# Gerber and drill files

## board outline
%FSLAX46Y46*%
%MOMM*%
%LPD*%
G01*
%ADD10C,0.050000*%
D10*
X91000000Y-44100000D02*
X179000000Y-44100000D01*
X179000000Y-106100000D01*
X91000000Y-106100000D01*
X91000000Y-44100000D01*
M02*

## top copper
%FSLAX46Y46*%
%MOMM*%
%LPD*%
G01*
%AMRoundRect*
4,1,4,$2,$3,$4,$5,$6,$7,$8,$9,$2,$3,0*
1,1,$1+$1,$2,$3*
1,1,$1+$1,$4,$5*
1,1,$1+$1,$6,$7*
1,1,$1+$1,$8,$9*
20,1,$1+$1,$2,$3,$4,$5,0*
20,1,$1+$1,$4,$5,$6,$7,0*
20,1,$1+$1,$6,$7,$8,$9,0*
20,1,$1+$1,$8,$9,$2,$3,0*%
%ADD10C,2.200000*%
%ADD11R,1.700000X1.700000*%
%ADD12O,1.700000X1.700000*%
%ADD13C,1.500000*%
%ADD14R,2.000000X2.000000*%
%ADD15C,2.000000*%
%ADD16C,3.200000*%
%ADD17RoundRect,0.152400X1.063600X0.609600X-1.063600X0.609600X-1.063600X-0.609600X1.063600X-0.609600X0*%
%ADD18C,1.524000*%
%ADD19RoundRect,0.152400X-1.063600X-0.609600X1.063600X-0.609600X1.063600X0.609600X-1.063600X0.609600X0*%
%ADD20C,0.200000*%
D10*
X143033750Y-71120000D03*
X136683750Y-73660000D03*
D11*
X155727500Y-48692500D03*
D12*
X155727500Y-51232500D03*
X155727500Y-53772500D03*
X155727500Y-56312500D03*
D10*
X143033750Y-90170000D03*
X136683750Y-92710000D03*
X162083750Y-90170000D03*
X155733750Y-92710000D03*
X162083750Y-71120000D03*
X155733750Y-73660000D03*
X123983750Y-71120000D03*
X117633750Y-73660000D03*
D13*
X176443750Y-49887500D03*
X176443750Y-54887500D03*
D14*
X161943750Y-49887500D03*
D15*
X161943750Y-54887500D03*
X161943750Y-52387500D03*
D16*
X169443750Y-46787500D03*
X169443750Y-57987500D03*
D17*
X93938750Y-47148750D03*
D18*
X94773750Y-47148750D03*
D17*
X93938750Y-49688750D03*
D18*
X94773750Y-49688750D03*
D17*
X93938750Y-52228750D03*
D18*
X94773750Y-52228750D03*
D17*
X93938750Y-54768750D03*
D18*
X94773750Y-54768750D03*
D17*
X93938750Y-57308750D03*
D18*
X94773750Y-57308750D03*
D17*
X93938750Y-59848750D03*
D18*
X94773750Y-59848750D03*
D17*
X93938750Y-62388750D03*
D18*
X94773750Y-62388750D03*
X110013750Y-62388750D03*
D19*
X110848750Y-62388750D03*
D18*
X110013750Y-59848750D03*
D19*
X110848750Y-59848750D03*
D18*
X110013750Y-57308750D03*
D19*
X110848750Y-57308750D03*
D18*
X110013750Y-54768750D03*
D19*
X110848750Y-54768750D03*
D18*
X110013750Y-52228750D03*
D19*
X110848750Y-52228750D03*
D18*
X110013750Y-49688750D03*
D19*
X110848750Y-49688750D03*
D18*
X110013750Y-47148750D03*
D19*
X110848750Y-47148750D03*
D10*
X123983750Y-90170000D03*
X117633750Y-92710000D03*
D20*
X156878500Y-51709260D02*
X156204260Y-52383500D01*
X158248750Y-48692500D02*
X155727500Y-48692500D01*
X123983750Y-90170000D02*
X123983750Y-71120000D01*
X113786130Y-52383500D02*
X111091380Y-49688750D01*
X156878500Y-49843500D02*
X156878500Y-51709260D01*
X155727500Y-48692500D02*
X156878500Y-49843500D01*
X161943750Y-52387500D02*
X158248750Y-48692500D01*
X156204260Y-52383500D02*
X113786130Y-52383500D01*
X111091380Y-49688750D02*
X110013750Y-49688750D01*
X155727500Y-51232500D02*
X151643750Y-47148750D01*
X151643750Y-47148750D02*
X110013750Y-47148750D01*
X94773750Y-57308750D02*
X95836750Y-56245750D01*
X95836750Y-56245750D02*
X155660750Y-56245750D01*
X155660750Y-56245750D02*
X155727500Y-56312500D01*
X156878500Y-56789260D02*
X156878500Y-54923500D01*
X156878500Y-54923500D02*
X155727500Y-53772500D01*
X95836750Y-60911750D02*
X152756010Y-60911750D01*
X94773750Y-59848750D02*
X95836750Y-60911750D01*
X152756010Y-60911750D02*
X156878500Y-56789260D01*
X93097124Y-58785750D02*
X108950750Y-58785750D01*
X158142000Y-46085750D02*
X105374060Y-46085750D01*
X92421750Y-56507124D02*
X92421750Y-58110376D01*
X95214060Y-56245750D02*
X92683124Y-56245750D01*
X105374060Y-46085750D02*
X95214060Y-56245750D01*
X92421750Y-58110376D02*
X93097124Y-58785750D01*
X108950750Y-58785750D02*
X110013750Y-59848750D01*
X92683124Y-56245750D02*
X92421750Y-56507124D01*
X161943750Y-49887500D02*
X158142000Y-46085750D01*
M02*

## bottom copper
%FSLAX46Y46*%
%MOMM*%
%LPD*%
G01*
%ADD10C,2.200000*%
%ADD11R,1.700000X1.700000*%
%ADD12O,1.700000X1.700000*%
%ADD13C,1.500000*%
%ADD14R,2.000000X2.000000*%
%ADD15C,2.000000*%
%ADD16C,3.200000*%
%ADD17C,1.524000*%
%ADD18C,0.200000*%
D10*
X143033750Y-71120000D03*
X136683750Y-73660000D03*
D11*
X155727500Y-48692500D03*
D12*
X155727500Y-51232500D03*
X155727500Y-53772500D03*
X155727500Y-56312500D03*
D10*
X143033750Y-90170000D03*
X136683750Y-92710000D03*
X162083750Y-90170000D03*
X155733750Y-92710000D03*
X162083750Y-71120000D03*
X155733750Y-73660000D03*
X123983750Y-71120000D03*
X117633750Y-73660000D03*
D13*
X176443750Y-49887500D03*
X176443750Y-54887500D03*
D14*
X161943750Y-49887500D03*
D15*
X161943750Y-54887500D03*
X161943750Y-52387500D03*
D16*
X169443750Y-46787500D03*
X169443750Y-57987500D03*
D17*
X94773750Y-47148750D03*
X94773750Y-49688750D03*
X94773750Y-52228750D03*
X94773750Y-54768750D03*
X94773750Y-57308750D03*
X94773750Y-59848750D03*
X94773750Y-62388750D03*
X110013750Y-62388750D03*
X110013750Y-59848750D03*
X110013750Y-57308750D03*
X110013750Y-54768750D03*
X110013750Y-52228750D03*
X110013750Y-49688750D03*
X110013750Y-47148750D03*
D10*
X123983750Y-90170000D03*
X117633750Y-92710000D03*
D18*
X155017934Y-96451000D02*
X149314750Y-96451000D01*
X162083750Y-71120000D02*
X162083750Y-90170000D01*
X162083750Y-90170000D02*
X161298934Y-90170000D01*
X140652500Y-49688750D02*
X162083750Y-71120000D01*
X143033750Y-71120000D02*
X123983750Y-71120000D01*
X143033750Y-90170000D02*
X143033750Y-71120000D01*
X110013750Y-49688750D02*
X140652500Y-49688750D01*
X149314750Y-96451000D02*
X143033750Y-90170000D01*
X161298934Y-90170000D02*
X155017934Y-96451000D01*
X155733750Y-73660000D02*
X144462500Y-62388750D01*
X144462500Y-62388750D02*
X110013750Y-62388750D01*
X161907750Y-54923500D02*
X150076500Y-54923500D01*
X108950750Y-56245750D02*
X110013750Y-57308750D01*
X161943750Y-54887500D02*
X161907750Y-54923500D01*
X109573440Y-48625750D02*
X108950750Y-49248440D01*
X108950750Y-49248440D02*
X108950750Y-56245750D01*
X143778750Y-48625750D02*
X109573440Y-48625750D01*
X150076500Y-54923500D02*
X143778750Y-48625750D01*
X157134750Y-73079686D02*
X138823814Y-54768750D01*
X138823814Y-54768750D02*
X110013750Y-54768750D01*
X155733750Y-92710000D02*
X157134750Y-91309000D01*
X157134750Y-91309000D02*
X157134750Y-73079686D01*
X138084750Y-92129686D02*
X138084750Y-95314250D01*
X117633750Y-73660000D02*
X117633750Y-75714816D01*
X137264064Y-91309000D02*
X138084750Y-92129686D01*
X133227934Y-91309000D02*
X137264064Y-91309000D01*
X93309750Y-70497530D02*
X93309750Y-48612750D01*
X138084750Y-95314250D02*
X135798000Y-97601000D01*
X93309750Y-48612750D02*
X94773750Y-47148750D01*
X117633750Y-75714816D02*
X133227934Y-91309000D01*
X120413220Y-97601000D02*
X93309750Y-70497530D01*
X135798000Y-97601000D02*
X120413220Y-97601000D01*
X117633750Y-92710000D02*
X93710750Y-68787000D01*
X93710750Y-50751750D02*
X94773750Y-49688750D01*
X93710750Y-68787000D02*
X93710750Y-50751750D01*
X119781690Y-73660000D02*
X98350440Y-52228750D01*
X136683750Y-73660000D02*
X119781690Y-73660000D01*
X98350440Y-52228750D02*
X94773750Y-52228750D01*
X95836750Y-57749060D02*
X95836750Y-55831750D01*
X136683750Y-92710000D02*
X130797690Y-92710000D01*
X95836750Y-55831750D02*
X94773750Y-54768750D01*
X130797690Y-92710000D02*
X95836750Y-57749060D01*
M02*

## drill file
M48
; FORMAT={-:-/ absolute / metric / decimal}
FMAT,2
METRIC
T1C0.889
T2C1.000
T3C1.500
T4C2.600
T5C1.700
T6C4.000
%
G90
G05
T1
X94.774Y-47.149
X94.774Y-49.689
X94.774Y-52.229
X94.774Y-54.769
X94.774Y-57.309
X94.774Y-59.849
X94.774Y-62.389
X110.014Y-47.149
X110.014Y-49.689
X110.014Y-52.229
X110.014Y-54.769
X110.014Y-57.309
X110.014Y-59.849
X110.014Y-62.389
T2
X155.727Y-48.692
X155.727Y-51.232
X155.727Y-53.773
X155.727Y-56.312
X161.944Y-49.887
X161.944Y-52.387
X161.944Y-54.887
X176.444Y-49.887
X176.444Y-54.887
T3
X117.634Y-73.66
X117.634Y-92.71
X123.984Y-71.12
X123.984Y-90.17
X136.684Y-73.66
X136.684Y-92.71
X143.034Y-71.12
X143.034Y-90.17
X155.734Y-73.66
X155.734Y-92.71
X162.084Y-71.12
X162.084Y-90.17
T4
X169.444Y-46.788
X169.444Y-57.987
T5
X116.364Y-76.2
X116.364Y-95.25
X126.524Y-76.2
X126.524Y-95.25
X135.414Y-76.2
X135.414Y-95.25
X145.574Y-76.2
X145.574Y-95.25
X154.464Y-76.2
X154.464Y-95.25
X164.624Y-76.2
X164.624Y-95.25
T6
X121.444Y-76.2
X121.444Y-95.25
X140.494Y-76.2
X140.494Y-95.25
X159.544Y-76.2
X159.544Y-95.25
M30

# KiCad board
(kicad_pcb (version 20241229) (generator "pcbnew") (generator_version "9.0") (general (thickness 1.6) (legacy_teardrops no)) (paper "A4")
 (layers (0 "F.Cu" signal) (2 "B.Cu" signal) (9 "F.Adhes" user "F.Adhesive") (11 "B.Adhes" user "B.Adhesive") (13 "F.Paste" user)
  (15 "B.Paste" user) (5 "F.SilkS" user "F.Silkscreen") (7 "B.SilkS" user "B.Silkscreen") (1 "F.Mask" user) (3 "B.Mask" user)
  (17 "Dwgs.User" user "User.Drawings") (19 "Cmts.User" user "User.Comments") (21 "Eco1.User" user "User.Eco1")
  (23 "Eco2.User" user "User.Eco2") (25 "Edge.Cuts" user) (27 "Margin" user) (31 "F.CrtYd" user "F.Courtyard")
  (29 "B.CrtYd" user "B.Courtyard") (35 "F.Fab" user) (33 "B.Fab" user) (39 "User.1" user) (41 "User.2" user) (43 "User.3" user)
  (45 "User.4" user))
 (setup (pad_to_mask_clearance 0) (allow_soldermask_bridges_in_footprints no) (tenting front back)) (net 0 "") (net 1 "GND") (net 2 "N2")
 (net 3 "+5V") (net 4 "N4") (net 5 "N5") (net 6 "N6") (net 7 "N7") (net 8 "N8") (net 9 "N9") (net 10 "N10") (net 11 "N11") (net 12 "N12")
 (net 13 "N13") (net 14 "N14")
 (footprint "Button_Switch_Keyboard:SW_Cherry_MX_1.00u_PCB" (layer "F.Cu") (at 143.03375 71.12)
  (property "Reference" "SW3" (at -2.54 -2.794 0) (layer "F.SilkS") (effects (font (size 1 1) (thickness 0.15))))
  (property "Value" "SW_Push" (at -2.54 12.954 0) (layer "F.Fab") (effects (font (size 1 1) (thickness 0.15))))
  (pad "" np_thru_hole circle (at -7.62 5.08) (size 1.7 1.7) (drill 1.7) (layers "*.Cu" "*.Mask"))
  (pad "" np_thru_hole circle (at -2.54 5.08) (size 4 4) (drill 4) (layers "*.Cu" "*.Mask"))
  (pad "" np_thru_hole circle (at 2.54 5.08) (size 1.7 1.7) (drill 1.7) (layers "*.Cu" "*.Mask"))
  (pad "1" thru_hole circle (at 0 0) (size 2.2 2.2) (drill 1.5) (layers "*.Cu" "*.Mask") (remove_unused_layers no) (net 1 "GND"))
  (pad "2" thru_hole circle (at -6.35 2.54) (size 2.2 2.2) (drill 1.5) (layers "*.Cu" "*.Mask") (remove_unused_layers no) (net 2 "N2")))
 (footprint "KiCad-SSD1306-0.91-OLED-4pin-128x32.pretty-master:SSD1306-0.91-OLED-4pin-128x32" (layer "F.Cu") (at 119.2275 46.5025)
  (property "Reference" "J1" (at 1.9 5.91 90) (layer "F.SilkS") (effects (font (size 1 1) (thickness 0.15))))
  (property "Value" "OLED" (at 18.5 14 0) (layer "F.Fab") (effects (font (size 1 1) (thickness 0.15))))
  (pad "1" thru_hole rect (at 36.5 2.19) (size 1.7 1.7) (drill 1) (layers "*.Cu" "*.Mask") (remove_unused_layers no) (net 1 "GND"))
  (pad "2" thru_hole oval (at 36.5 4.73) (size 1.7 1.7) (drill 1) (layers "*.Cu" "*.Mask") (remove_unused_layers no) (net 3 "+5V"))
  (pad "3" thru_hole oval (at 36.5 7.27) (size 1.7 1.7) (drill 1) (layers "*.Cu" "*.Mask") (remove_unused_layers no) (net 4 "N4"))
  (pad "4" thru_hole oval (at 36.5 9.81) (size 1.7 1.7) (drill 1) (layers "*.Cu" "*.Mask") (remove_unused_layers no) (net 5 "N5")))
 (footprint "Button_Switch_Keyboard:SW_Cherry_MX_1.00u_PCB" (layer "F.Cu") (at 143.03375 90.17)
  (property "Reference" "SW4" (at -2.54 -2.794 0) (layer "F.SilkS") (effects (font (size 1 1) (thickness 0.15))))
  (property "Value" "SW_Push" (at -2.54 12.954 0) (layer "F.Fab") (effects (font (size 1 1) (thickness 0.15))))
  (pad "" np_thru_hole circle (at -7.62 5.08) (size 1.7 1.7) (drill 1.7) (layers "*.Cu" "*.Mask"))
  (pad "" np_thru_hole circle (at -2.54 5.08) (size 4 4) (drill 4) (layers "*.Cu" "*.Mask"))
  (pad "" np_thru_hole circle (at 2.54 5.08) (size 1.7 1.7) (drill 1.7) (layers "*.Cu" "*.Mask"))
  (pad "1" thru_hole circle (at 0 0) (size 2.2 2.2) (drill 1.5) (layers "*.Cu" "*.Mask") (remove_unused_layers no) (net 1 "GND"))
  (pad "2" thru_hole circle (at -6.35 2.54) (size 2.2 2.2) (drill 1.5) (layers "*.Cu" "*.Mask") (remove_unused_layers no) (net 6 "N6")))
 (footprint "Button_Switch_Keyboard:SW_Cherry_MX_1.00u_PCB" (layer "F.Cu") (at 162.08375 90.17)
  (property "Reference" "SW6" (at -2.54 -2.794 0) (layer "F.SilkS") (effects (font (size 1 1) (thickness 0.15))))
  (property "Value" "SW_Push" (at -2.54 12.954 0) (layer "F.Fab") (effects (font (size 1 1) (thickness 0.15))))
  (pad "" np_thru_hole circle (at -7.62 5.08) (size 1.7 1.7) (drill 1.7) (layers "*.Cu" "*.Mask"))
  (pad "" np_thru_hole circle (at -2.54 5.08) (size 4 4) (drill 4) (layers "*.Cu" "*.Mask"))
  (pad "" np_thru_hole circle (at 2.54 5.08) (size 1.7 1.7) (drill 1.7) (layers "*.Cu" "*.Mask"))
  (pad "1" thru_hole circle (at 0 0) (size 2.2 2.2) (drill 1.5) (layers "*.Cu" "*.Mask") (remove_unused_layers no) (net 1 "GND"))
  (pad "2" thru_hole circle (at -6.35 2.54) (size 2.2 2.2) (drill 1.5) (layers "*.Cu" "*.Mask") (remove_unused_layers no) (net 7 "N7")))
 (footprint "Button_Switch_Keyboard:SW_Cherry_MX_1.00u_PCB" (layer "F.Cu") (at 162.08375 71.12)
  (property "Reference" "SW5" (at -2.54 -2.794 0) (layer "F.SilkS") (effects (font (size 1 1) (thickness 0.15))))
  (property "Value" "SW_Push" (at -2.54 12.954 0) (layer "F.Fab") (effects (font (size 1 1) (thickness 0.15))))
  (pad "" np_thru_hole circle (at -7.62 5.08) (size 1.7 1.7) (drill 1.7) (layers "*.Cu" "*.Mask"))
  (pad "" np_thru_hole circle (at -2.54 5.08) (size 4 4) (drill 4) (layers "*.Cu" "*.Mask"))
  (pad "" np_thru_hole circle (at 2.54 5.08) (size 1.7 1.7) (drill 1.7) (layers "*.Cu" "*.Mask"))
  (pad "1" thru_hole circle (at 0 0) (size 2.2 2.2) (drill 1.5) (layers "*.Cu" "*.Mask") (remove_unused_layers no) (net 1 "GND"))
  (pad "2" thru_hole circle (at -6.35 2.54) (size 2.2 2.2) (drill 1.5) (layers "*.Cu" "*.Mask") (remove_unused_layers no) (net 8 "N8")))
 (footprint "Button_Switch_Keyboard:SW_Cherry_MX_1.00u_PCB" (layer "F.Cu") (at 123.98375 71.12)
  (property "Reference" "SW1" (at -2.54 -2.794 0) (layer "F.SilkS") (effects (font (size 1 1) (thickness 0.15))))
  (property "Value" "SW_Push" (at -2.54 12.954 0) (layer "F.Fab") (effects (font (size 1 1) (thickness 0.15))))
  (pad "" np_thru_hole circle (at -7.62 5.08) (size 1.7 1.7) (drill 1.7) (layers "*.Cu" "*.Mask"))
  (pad "" np_thru_hole circle (at -2.54 5.08) (size 4 4) (drill 4) (layers "*.Cu" "*.Mask"))
  (pad "" np_thru_hole circle (at 2.54 5.08) (size 1.7 1.7) (drill 1.7) (layers "*.Cu" "*.Mask"))
  (pad "1" thru_hole circle (at 0 0) (size 2.2 2.2) (drill 1.5) (layers "*.Cu" "*.Mask") (remove_unused_layers no) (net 1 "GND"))
  (pad "2" thru_hole circle (at -6.35 2.54) (size 2.2 2.2) (drill 1.5) (layers "*.Cu" "*.Mask") (remove_unused_layers no) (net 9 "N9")))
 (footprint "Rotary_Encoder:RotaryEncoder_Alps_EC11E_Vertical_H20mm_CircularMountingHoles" (layer "F.Cu") (at 161.94375 49.8875)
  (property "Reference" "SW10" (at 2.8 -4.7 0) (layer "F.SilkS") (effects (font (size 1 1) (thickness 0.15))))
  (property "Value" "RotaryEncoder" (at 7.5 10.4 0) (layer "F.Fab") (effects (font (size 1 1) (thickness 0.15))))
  (pad "" thru_hole circle (at 14.5 0) (size 1.5 1.5) (drill 1) (layers "*.Cu" "*.Mask") (remove_unused_layers no))
  (pad "" thru_hole circle (at 14.5 5) (size 1.5 1.5) (drill 1) (layers "*.Cu" "*.Mask") (remove_unused_layers no))
  (pad "A" thru_hole rect (at 0 0) (size 2 2) (drill 1) (layers "*.Cu" "*.Mask") (remove_unused_layers no) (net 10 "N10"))
  (pad "B" thru_hole circle (at 0 5) (size 2 2) (drill 1) (layers "*.Cu" "*.Mask") (remove_unused_layers no) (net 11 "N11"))
  (pad "C" thru_hole circle (at 0 2.5) (size 2 2) (drill 1) (layers "*.Cu" "*.Mask") (remove_unused_layers no) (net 1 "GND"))
  (pad "MP" thru_hole circle (at 7.5 -3.1) (size 3.2 3.2) (drill 2.6) (layers "*.Cu" "*.Mask") (remove_unused_layers no))
  (pad "MP" thru_hole circle (at 7.5 8.1) (size 3.2 3.2) (drill 2.6) (layers "*.Cu" "*.Mask") (remove_unused_layers no)))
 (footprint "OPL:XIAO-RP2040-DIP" (layer "F.Cu") (at 102.39375 54.76875)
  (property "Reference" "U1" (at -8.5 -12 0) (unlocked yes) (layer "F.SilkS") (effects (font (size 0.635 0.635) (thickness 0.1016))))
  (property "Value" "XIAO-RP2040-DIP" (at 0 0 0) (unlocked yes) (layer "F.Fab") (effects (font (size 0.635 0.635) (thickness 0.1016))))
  (pad "1" smd roundrect (at -8.455 -7.62 180) (size 2.432 1.524) (layers "F.Cu" "F.Mask") (roundrect_rratio 0.1) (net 9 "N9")
   (thermal_bridge_angle 45))
  (pad "1" thru_hole circle (at -7.62 -7.62 180) (size 1.524 1.524) (drill 0.889) (layers "*.Cu" "*.Mask") (remove_unused_layers no)
   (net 9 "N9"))
  (pad "2" smd roundrect (at -8.455 -5.08 180) (size 2.432 1.524) (layers "F.Cu" "F.Mask") (roundrect_rratio 0.1) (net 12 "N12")
   (thermal_bridge_angle 45))
  (pad "2" thru_hole circle (at -7.62 -5.08 180) (size 1.524 1.524) (drill 0.889) (layers "*.Cu" "*.Mask") (remove_unused_layers no)
   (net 12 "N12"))
  (pad "3" smd roundrect (at -8.455 -2.54 180) (size 2.432 1.524) (layers "F.Cu" "F.Mask") (roundrect_rratio 0.1) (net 2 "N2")
   (thermal_bridge_angle 45))
  (pad "3" thru_hole circle (at -7.62 -2.54 180) (size 1.524 1.524) (drill 0.889) (layers "*.Cu" "*.Mask") (remove_unused_layers no)
   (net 2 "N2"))
  (pad "4" smd roundrect (at -8.455 0 180) (size 2.432 1.524) (layers "F.Cu" "F.Mask") (roundrect_rratio 0.1) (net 6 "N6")
   (thermal_bridge_angle 45))
  (pad "4" thru_hole circle (at -7.62 0 180) (size 1.524 1.524) (drill 0.889) (layers "*.Cu" "*.Mask") (remove_unused_layers no)
   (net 6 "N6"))
  (pad "5" smd roundrect (at -8.455 2.54 180) (size 2.432 1.524) (layers "F.Cu" "F.Mask") (roundrect_rratio 0.1) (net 5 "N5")
   (thermal_bridge_angle 45))
  (pad "5" thru_hole circle (at -7.62 2.54 180) (size 1.524 1.524) (drill 0.889) (layers "*.Cu" "*.Mask") (remove_unused_layers no)
   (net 5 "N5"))
  (pad "6" smd roundrect (at -8.455 5.08 180) (size 2.432 1.524) (layers "F.Cu" "F.Mask") (roundrect_rratio 0.1) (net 4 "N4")
   (thermal_bridge_angle 45))
  (pad "6" thru_hole circle (at -7.62 5.08 180) (size 1.524 1.524) (drill 0.889) (layers "*.Cu" "*.Mask") (remove_unused_layers no)
   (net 4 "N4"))
  (pad "7" smd roundrect (at -8.455 7.62 180) (size 2.432 1.524) (layers "F.Cu" "F.Mask") (roundrect_rratio 0.1) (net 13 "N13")
   (thermal_bridge_angle 45))
  (pad "7" thru_hole circle (at -7.62 7.62 180) (size 1.524 1.524) (drill 0.889) (layers "*.Cu" "*.Mask") (remove_unused_layers no)
   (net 13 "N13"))
  (pad "8" thru_hole circle (at 7.62 7.62) (size 1.524 1.524) (drill 0.889) (layers "*.Cu" "*.Mask") (remove_unused_layers no) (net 8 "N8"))
  (pad "8" smd roundrect (at 8.455 7.62) (size 2.432 1.524) (layers "F.Cu" "F.Mask") (roundrect_rratio 0.1) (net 8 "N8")
   (thermal_bridge_angle 45))
  (pad "9" thru_hole circle (at 7.62 5.08) (size 1.524 1.524) (drill 0.889) (layers "*.Cu" "*.Mask") (remove_unused_layers no)
   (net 10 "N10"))
  (pad "9" smd roundrect (at 8.455 5.08) (size 2.432 1.524) (layers "F.Cu" "F.Mask") (roundrect_rratio 0.1) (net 10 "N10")
   (thermal_bridge_angle 45))
  (pad "10" thru_hole circle (at 7.62 2.54) (size 1.524 1.524) (drill 0.889) (layers "*.Cu" "*.Mask") (remove_unused_layers no)
   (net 11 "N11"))
  (pad "10" smd roundrect (at 8.455 2.54) (size 2.432 1.524) (layers "F.Cu" "F.Mask") (roundrect_rratio 0.1) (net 11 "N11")
   (thermal_bridge_angle 45))
  (pad "11" thru_hole circle (at 7.62 0) (size 1.524 1.524) (drill 0.889) (layers "*.Cu" "*.Mask") (remove_unused_layers no) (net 7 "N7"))
  (pad "11" smd roundrect (at 8.455 0) (size 2.432 1.524) (layers "F.Cu" "F.Mask") (roundrect_rratio 0.1) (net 7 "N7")
   (thermal_bridge_angle 45))
  (pad "12" thru_hole circle (at 7.62 -2.54) (size 1.524 1.524) (drill 0.889) (layers "*.Cu" "*.Mask") (remove_unused_layers no)
   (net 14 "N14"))
  (pad "12" smd roundrect (at 8.455 -2.54) (size 2.432 1.524) (layers "F.Cu" "F.Mask") (roundrect_rratio 0.1) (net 14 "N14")
   (thermal_bridge_angle 45))
  (pad "13" thru_hole circle (at 7.62 -5.08) (size 1.524 1.524) (drill 0.889) (layers "*.Cu" "*.Mask") (remove_unused_layers no)
   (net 1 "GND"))
  (pad "13" smd roundrect (at 8.455 -5.08) (size 2.432 1.524) (layers "F.Cu" "F.Mask") (roundrect_rratio 0.1) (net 1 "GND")
   (thermal_bridge_angle 45))
  (pad "14" thru_hole circle (at 7.62 -7.62) (size 1.524 1.524) (drill 0.889) (layers "*.Cu" "*.Mask") (remove_unused_layers no)
   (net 3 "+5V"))
  (pad "14" smd roundrect (at 8.455 -7.62) (size 2.432 1.524) (layers "F.Cu" "F.Mask") (roundrect_rratio 0.1) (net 3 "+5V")
   (thermal_bridge_angle 45)))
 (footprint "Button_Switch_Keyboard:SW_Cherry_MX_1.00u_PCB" (layer "F.Cu") (at 123.98375 90.17)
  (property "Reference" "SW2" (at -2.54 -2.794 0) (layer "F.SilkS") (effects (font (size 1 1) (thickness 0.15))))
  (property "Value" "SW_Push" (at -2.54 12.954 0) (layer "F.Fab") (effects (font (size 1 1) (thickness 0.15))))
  (pad "" np_thru_hole circle (at -7.62 5.08) (size 1.7 1.7) (drill 1.7) (layers "*.Cu" "*.Mask"))
  (pad "" np_thru_hole circle (at -2.54 5.08) (size 4 4) (drill 4) (layers "*.Cu" "*.Mask"))
  (pad "" np_thru_hole circle (at 2.54 5.08) (size 1.7 1.7) (drill 1.7) (layers "*.Cu" "*.Mask"))
  (pad "1" thru_hole circle (at 0 0) (size 2.2 2.2) (drill 1.5) (layers "*.Cu" "*.Mask") (remove_unused_layers no) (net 1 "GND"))
  (pad "2" thru_hole circle (at -6.35 2.54) (size 2.2 2.2) (drill 1.5) (layers "*.Cu" "*.Mask") (remove_unused_layers no) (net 12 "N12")))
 (gr_rect (start 91 44.1) (end 179 106.1) (stroke (width 0.05) (type default)) (fill no) (layer "Edge.Cuts"))
 (segment (start 156.8785 51.70926) (end 156.20426 52.3835) (width 0.2) (layer "F.Cu") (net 1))
 (segment (start 158.24875 48.6925) (end 155.7275 48.6925) (width 0.2) (layer "F.Cu") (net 1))
 (segment (start 123.98375 90.17) (end 123.98375 71.12) (width 0.2) (layer "F.Cu") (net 1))
 (segment (start 113.78613 52.3835) (end 111.09138 49.68875) (width 0.2) (layer "F.Cu") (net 1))
 (segment (start 156.8785 49.8435) (end 156.8785 51.70926) (width 0.2) (layer "F.Cu") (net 1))
 (segment (start 155.7275 48.6925) (end 156.8785 49.8435) (width 0.2) (layer "F.Cu") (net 1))
 (segment (start 161.94375 52.3875) (end 158.24875 48.6925) (width 0.2) (layer "F.Cu") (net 1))
 (segment (start 156.20426 52.3835) (end 113.78613 52.3835) (width 0.2) (layer "F.Cu") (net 1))
 (segment (start 111.09138 49.68875) (end 110.01375 49.68875) (width 0.2) (layer "F.Cu") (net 1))
 (segment (start 155.017934 96.451) (end 149.31475 96.451) (width 0.2) (layer "B.Cu") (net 1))
 (segment (start 162.08375 71.12) (end 162.08375 90.17) (width 0.2) (layer "B.Cu") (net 1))
 (segment (start 162.08375 90.17) (end 161.298934 90.17) (width 0.2) (layer "B.Cu") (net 1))
 (segment (start 140.6525 49.68875) (end 162.08375 71.12) (width 0.2) (layer "B.Cu") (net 1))
 (segment (start 143.03375 71.12) (end 123.98375 71.12) (width 0.2) (layer "B.Cu") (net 1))
 (segment (start 143.03375 90.17) (end 143.03375 71.12) (width 0.2) (layer "B.Cu") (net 1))
 (segment (start 110.01375 49.68875) (end 140.6525 49.68875) (width 0.2) (layer "B.Cu") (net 1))
 (segment (start 149.31475 96.451) (end 143.03375 90.17) (width 0.2) (layer "B.Cu") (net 1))
 (segment (start 161.298934 90.17) (end 155.017934 96.451) (width 0.2) (layer "B.Cu") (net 1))
 (segment (start 155.7275 51.2325) (end 151.64375 47.14875) (width 0.2) (layer "F.Cu") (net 3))
 (segment (start 151.64375 47.14875) (end 110.01375 47.14875) (width 0.2) (layer "F.Cu") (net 3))
 (segment (start 155.73375 73.66) (end 144.4625 62.38875) (width 0.2) (layer "B.Cu") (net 8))
 (segment (start 144.4625 62.38875) (end 110.01375 62.38875) (width 0.2) (layer "B.Cu") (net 8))
 (segment (start 94.77375 57.30875) (end 95.83675 56.24575) (width 0.2) (layer "F.Cu") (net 5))
 (segment (start 95.83675 56.24575) (end 155.66075 56.24575) (width 0.2) (layer "F.Cu") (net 5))
 (segment (start 155.66075 56.24575) (end 155.7275 56.3125) (width 0.2) (layer "F.Cu") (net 5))
 (segment (start 161.90775 54.9235) (end 150.0765 54.9235) (width 0.2) (layer "B.Cu") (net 11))
 (segment (start 108.95075 56.24575) (end 110.01375 57.30875) (width 0.2) (layer "B.Cu") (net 11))
 (segment (start 161.94375 54.8875) (end 161.90775 54.9235) (width 0.2) (layer "B.Cu") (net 11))
 (segment (start 109.57344 48.62575) (end 108.95075 49.24844) (width 0.2) (layer "B.Cu") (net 11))
 (segment (start 108.95075 49.24844) (end 108.95075 56.24575) (width 0.2) (layer "B.Cu") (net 11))
 (segment (start 143.77875 48.62575) (end 109.57344 48.62575) (width 0.2) (layer "B.Cu") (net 11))
 (segment (start 150.0765 54.9235) (end 143.77875 48.62575) (width 0.2) (layer "B.Cu") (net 11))
 (segment (start 157.13475 73.079686) (end 138.823814 54.76875) (width 0.2) (layer "B.Cu") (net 7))
 (segment (start 138.823814 54.76875) (end 110.01375 54.76875) (width 0.2) (layer "B.Cu") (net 7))
 (segment (start 155.73375 92.71) (end 157.13475 91.309) (width 0.2) (layer "B.Cu") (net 7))
 (segment (start 157.13475 91.309) (end 157.13475 73.079686) (width 0.2) (layer "B.Cu") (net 7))
 (segment (start 156.8785 56.78926) (end 156.8785 54.9235) (width 0.2) (layer "F.Cu") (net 4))
 (segment (start 156.8785 54.9235) (end 155.7275 53.7725) (width 0.2) (layer "F.Cu") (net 4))
 (segment (start 95.83675 60.91175) (end 152.75601 60.91175) (width 0.2) (layer "F.Cu") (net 4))
 (segment (start 94.77375 59.84875) (end 95.83675 60.91175) (width 0.2) (layer "F.Cu") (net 4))
 (segment (start 152.75601 60.91175) (end 156.8785 56.78926) (width 0.2) (layer "F.Cu") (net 4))
 (segment (start 138.08475 92.129686) (end 138.08475 95.31425) (width 0.2) (layer "B.Cu") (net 9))
 (segment (start 117.63375 73.66) (end 117.63375 75.714816) (width 0.2) (layer "B.Cu") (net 9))
 (segment (start 137.264064 91.309) (end 138.08475 92.129686) (width 0.2) (layer "B.Cu") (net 9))
 (segment (start 133.227934 91.309) (end 137.264064 91.309) (width 0.2) (layer "B.Cu") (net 9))
 (segment (start 93.30975 70.49753) (end 93.30975 48.61275) (width 0.2) (layer "B.Cu") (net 9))
 (segment (start 138.08475 95.31425) (end 135.798 97.601) (width 0.2) (layer "B.Cu") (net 9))
 (segment (start 93.30975 48.61275) (end 94.77375 47.14875) (width 0.2) (layer "B.Cu") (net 9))
 (segment (start 117.63375 75.714816) (end 133.227934 91.309) (width 0.2) (layer "B.Cu") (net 9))
 (segment (start 120.41322 97.601) (end 93.30975 70.49753) (width 0.2) (layer "B.Cu") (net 9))
 (segment (start 135.798 97.601) (end 120.41322 97.601) (width 0.2) (layer "B.Cu") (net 9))
 (segment (start 117.63375 92.71) (end 93.71075 68.787) (width 0.2) (layer "B.Cu") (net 12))
 (segment (start 93.71075 50.75175) (end 94.77375 49.68875) (width 0.2) (layer "B.Cu") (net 12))
 (segment (start 93.71075 68.787) (end 93.71075 50.75175) (width 0.2) (layer "B.Cu") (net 12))
 (segment (start 119.78169 73.66) (end 98.35044 52.22875) (width 0.2) (layer "B.Cu") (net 2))
 (segment (start 136.68375 73.66) (end 119.78169 73.66) (width 0.2) (layer "B.Cu") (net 2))
 (segment (start 98.35044 52.22875) (end 94.77375 52.22875) (width 0.2) (layer "B.Cu") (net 2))
 (segment (start 95.83675 57.74906) (end 95.83675 55.83175) (width 0.2) (layer "B.Cu") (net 6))
 (segment (start 136.68375 92.71) (end 130.79769 92.71) (width 0.2) (layer "B.Cu") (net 6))
 (segment (start 95.83675 55.83175) (end 94.77375 54.76875) (width 0.2) (layer "B.Cu") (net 6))
 (segment (start 130.79769 92.71) (end 95.83675 57.74906) (width 0.2) (layer "B.Cu") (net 6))
 (segment (start 93.097124 58.78575) (end 108.95075 58.78575) (width 0.2) (layer "F.Cu") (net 10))
 (segment (start 158.142 46.08575) (end 105.37406 46.08575) (width 0.2) (layer "F.Cu") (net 10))
 (segment (start 92.42175 56.507124) (end 92.42175 58.110376) (width 0.2) (layer "F.Cu") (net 10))
 (segment (start 95.21406 56.24575) (end 92.683124 56.24575) (width 0.2) (layer "F.Cu") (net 10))
 (segment (start 105.37406 46.08575) (end 95.21406 56.24575) (width 0.2) (layer "F.Cu") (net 10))
 (segment (start 92.42175 58.110376) (end 93.097124 58.78575) (width 0.2) (layer "F.Cu") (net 10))
 (segment (start 108.95075 58.78575) (end 110.01375 59.84875) (width 0.2) (layer "F.Cu") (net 10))
 (segment (start 92.683124 56.24575) (end 92.42175 56.507124) (width 0.2) (layer "F.Cu") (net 10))
 (segment (start 161.94375 49.8875) (end 158.142 46.08575) (width 0.2) (layer "F.Cu") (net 10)))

